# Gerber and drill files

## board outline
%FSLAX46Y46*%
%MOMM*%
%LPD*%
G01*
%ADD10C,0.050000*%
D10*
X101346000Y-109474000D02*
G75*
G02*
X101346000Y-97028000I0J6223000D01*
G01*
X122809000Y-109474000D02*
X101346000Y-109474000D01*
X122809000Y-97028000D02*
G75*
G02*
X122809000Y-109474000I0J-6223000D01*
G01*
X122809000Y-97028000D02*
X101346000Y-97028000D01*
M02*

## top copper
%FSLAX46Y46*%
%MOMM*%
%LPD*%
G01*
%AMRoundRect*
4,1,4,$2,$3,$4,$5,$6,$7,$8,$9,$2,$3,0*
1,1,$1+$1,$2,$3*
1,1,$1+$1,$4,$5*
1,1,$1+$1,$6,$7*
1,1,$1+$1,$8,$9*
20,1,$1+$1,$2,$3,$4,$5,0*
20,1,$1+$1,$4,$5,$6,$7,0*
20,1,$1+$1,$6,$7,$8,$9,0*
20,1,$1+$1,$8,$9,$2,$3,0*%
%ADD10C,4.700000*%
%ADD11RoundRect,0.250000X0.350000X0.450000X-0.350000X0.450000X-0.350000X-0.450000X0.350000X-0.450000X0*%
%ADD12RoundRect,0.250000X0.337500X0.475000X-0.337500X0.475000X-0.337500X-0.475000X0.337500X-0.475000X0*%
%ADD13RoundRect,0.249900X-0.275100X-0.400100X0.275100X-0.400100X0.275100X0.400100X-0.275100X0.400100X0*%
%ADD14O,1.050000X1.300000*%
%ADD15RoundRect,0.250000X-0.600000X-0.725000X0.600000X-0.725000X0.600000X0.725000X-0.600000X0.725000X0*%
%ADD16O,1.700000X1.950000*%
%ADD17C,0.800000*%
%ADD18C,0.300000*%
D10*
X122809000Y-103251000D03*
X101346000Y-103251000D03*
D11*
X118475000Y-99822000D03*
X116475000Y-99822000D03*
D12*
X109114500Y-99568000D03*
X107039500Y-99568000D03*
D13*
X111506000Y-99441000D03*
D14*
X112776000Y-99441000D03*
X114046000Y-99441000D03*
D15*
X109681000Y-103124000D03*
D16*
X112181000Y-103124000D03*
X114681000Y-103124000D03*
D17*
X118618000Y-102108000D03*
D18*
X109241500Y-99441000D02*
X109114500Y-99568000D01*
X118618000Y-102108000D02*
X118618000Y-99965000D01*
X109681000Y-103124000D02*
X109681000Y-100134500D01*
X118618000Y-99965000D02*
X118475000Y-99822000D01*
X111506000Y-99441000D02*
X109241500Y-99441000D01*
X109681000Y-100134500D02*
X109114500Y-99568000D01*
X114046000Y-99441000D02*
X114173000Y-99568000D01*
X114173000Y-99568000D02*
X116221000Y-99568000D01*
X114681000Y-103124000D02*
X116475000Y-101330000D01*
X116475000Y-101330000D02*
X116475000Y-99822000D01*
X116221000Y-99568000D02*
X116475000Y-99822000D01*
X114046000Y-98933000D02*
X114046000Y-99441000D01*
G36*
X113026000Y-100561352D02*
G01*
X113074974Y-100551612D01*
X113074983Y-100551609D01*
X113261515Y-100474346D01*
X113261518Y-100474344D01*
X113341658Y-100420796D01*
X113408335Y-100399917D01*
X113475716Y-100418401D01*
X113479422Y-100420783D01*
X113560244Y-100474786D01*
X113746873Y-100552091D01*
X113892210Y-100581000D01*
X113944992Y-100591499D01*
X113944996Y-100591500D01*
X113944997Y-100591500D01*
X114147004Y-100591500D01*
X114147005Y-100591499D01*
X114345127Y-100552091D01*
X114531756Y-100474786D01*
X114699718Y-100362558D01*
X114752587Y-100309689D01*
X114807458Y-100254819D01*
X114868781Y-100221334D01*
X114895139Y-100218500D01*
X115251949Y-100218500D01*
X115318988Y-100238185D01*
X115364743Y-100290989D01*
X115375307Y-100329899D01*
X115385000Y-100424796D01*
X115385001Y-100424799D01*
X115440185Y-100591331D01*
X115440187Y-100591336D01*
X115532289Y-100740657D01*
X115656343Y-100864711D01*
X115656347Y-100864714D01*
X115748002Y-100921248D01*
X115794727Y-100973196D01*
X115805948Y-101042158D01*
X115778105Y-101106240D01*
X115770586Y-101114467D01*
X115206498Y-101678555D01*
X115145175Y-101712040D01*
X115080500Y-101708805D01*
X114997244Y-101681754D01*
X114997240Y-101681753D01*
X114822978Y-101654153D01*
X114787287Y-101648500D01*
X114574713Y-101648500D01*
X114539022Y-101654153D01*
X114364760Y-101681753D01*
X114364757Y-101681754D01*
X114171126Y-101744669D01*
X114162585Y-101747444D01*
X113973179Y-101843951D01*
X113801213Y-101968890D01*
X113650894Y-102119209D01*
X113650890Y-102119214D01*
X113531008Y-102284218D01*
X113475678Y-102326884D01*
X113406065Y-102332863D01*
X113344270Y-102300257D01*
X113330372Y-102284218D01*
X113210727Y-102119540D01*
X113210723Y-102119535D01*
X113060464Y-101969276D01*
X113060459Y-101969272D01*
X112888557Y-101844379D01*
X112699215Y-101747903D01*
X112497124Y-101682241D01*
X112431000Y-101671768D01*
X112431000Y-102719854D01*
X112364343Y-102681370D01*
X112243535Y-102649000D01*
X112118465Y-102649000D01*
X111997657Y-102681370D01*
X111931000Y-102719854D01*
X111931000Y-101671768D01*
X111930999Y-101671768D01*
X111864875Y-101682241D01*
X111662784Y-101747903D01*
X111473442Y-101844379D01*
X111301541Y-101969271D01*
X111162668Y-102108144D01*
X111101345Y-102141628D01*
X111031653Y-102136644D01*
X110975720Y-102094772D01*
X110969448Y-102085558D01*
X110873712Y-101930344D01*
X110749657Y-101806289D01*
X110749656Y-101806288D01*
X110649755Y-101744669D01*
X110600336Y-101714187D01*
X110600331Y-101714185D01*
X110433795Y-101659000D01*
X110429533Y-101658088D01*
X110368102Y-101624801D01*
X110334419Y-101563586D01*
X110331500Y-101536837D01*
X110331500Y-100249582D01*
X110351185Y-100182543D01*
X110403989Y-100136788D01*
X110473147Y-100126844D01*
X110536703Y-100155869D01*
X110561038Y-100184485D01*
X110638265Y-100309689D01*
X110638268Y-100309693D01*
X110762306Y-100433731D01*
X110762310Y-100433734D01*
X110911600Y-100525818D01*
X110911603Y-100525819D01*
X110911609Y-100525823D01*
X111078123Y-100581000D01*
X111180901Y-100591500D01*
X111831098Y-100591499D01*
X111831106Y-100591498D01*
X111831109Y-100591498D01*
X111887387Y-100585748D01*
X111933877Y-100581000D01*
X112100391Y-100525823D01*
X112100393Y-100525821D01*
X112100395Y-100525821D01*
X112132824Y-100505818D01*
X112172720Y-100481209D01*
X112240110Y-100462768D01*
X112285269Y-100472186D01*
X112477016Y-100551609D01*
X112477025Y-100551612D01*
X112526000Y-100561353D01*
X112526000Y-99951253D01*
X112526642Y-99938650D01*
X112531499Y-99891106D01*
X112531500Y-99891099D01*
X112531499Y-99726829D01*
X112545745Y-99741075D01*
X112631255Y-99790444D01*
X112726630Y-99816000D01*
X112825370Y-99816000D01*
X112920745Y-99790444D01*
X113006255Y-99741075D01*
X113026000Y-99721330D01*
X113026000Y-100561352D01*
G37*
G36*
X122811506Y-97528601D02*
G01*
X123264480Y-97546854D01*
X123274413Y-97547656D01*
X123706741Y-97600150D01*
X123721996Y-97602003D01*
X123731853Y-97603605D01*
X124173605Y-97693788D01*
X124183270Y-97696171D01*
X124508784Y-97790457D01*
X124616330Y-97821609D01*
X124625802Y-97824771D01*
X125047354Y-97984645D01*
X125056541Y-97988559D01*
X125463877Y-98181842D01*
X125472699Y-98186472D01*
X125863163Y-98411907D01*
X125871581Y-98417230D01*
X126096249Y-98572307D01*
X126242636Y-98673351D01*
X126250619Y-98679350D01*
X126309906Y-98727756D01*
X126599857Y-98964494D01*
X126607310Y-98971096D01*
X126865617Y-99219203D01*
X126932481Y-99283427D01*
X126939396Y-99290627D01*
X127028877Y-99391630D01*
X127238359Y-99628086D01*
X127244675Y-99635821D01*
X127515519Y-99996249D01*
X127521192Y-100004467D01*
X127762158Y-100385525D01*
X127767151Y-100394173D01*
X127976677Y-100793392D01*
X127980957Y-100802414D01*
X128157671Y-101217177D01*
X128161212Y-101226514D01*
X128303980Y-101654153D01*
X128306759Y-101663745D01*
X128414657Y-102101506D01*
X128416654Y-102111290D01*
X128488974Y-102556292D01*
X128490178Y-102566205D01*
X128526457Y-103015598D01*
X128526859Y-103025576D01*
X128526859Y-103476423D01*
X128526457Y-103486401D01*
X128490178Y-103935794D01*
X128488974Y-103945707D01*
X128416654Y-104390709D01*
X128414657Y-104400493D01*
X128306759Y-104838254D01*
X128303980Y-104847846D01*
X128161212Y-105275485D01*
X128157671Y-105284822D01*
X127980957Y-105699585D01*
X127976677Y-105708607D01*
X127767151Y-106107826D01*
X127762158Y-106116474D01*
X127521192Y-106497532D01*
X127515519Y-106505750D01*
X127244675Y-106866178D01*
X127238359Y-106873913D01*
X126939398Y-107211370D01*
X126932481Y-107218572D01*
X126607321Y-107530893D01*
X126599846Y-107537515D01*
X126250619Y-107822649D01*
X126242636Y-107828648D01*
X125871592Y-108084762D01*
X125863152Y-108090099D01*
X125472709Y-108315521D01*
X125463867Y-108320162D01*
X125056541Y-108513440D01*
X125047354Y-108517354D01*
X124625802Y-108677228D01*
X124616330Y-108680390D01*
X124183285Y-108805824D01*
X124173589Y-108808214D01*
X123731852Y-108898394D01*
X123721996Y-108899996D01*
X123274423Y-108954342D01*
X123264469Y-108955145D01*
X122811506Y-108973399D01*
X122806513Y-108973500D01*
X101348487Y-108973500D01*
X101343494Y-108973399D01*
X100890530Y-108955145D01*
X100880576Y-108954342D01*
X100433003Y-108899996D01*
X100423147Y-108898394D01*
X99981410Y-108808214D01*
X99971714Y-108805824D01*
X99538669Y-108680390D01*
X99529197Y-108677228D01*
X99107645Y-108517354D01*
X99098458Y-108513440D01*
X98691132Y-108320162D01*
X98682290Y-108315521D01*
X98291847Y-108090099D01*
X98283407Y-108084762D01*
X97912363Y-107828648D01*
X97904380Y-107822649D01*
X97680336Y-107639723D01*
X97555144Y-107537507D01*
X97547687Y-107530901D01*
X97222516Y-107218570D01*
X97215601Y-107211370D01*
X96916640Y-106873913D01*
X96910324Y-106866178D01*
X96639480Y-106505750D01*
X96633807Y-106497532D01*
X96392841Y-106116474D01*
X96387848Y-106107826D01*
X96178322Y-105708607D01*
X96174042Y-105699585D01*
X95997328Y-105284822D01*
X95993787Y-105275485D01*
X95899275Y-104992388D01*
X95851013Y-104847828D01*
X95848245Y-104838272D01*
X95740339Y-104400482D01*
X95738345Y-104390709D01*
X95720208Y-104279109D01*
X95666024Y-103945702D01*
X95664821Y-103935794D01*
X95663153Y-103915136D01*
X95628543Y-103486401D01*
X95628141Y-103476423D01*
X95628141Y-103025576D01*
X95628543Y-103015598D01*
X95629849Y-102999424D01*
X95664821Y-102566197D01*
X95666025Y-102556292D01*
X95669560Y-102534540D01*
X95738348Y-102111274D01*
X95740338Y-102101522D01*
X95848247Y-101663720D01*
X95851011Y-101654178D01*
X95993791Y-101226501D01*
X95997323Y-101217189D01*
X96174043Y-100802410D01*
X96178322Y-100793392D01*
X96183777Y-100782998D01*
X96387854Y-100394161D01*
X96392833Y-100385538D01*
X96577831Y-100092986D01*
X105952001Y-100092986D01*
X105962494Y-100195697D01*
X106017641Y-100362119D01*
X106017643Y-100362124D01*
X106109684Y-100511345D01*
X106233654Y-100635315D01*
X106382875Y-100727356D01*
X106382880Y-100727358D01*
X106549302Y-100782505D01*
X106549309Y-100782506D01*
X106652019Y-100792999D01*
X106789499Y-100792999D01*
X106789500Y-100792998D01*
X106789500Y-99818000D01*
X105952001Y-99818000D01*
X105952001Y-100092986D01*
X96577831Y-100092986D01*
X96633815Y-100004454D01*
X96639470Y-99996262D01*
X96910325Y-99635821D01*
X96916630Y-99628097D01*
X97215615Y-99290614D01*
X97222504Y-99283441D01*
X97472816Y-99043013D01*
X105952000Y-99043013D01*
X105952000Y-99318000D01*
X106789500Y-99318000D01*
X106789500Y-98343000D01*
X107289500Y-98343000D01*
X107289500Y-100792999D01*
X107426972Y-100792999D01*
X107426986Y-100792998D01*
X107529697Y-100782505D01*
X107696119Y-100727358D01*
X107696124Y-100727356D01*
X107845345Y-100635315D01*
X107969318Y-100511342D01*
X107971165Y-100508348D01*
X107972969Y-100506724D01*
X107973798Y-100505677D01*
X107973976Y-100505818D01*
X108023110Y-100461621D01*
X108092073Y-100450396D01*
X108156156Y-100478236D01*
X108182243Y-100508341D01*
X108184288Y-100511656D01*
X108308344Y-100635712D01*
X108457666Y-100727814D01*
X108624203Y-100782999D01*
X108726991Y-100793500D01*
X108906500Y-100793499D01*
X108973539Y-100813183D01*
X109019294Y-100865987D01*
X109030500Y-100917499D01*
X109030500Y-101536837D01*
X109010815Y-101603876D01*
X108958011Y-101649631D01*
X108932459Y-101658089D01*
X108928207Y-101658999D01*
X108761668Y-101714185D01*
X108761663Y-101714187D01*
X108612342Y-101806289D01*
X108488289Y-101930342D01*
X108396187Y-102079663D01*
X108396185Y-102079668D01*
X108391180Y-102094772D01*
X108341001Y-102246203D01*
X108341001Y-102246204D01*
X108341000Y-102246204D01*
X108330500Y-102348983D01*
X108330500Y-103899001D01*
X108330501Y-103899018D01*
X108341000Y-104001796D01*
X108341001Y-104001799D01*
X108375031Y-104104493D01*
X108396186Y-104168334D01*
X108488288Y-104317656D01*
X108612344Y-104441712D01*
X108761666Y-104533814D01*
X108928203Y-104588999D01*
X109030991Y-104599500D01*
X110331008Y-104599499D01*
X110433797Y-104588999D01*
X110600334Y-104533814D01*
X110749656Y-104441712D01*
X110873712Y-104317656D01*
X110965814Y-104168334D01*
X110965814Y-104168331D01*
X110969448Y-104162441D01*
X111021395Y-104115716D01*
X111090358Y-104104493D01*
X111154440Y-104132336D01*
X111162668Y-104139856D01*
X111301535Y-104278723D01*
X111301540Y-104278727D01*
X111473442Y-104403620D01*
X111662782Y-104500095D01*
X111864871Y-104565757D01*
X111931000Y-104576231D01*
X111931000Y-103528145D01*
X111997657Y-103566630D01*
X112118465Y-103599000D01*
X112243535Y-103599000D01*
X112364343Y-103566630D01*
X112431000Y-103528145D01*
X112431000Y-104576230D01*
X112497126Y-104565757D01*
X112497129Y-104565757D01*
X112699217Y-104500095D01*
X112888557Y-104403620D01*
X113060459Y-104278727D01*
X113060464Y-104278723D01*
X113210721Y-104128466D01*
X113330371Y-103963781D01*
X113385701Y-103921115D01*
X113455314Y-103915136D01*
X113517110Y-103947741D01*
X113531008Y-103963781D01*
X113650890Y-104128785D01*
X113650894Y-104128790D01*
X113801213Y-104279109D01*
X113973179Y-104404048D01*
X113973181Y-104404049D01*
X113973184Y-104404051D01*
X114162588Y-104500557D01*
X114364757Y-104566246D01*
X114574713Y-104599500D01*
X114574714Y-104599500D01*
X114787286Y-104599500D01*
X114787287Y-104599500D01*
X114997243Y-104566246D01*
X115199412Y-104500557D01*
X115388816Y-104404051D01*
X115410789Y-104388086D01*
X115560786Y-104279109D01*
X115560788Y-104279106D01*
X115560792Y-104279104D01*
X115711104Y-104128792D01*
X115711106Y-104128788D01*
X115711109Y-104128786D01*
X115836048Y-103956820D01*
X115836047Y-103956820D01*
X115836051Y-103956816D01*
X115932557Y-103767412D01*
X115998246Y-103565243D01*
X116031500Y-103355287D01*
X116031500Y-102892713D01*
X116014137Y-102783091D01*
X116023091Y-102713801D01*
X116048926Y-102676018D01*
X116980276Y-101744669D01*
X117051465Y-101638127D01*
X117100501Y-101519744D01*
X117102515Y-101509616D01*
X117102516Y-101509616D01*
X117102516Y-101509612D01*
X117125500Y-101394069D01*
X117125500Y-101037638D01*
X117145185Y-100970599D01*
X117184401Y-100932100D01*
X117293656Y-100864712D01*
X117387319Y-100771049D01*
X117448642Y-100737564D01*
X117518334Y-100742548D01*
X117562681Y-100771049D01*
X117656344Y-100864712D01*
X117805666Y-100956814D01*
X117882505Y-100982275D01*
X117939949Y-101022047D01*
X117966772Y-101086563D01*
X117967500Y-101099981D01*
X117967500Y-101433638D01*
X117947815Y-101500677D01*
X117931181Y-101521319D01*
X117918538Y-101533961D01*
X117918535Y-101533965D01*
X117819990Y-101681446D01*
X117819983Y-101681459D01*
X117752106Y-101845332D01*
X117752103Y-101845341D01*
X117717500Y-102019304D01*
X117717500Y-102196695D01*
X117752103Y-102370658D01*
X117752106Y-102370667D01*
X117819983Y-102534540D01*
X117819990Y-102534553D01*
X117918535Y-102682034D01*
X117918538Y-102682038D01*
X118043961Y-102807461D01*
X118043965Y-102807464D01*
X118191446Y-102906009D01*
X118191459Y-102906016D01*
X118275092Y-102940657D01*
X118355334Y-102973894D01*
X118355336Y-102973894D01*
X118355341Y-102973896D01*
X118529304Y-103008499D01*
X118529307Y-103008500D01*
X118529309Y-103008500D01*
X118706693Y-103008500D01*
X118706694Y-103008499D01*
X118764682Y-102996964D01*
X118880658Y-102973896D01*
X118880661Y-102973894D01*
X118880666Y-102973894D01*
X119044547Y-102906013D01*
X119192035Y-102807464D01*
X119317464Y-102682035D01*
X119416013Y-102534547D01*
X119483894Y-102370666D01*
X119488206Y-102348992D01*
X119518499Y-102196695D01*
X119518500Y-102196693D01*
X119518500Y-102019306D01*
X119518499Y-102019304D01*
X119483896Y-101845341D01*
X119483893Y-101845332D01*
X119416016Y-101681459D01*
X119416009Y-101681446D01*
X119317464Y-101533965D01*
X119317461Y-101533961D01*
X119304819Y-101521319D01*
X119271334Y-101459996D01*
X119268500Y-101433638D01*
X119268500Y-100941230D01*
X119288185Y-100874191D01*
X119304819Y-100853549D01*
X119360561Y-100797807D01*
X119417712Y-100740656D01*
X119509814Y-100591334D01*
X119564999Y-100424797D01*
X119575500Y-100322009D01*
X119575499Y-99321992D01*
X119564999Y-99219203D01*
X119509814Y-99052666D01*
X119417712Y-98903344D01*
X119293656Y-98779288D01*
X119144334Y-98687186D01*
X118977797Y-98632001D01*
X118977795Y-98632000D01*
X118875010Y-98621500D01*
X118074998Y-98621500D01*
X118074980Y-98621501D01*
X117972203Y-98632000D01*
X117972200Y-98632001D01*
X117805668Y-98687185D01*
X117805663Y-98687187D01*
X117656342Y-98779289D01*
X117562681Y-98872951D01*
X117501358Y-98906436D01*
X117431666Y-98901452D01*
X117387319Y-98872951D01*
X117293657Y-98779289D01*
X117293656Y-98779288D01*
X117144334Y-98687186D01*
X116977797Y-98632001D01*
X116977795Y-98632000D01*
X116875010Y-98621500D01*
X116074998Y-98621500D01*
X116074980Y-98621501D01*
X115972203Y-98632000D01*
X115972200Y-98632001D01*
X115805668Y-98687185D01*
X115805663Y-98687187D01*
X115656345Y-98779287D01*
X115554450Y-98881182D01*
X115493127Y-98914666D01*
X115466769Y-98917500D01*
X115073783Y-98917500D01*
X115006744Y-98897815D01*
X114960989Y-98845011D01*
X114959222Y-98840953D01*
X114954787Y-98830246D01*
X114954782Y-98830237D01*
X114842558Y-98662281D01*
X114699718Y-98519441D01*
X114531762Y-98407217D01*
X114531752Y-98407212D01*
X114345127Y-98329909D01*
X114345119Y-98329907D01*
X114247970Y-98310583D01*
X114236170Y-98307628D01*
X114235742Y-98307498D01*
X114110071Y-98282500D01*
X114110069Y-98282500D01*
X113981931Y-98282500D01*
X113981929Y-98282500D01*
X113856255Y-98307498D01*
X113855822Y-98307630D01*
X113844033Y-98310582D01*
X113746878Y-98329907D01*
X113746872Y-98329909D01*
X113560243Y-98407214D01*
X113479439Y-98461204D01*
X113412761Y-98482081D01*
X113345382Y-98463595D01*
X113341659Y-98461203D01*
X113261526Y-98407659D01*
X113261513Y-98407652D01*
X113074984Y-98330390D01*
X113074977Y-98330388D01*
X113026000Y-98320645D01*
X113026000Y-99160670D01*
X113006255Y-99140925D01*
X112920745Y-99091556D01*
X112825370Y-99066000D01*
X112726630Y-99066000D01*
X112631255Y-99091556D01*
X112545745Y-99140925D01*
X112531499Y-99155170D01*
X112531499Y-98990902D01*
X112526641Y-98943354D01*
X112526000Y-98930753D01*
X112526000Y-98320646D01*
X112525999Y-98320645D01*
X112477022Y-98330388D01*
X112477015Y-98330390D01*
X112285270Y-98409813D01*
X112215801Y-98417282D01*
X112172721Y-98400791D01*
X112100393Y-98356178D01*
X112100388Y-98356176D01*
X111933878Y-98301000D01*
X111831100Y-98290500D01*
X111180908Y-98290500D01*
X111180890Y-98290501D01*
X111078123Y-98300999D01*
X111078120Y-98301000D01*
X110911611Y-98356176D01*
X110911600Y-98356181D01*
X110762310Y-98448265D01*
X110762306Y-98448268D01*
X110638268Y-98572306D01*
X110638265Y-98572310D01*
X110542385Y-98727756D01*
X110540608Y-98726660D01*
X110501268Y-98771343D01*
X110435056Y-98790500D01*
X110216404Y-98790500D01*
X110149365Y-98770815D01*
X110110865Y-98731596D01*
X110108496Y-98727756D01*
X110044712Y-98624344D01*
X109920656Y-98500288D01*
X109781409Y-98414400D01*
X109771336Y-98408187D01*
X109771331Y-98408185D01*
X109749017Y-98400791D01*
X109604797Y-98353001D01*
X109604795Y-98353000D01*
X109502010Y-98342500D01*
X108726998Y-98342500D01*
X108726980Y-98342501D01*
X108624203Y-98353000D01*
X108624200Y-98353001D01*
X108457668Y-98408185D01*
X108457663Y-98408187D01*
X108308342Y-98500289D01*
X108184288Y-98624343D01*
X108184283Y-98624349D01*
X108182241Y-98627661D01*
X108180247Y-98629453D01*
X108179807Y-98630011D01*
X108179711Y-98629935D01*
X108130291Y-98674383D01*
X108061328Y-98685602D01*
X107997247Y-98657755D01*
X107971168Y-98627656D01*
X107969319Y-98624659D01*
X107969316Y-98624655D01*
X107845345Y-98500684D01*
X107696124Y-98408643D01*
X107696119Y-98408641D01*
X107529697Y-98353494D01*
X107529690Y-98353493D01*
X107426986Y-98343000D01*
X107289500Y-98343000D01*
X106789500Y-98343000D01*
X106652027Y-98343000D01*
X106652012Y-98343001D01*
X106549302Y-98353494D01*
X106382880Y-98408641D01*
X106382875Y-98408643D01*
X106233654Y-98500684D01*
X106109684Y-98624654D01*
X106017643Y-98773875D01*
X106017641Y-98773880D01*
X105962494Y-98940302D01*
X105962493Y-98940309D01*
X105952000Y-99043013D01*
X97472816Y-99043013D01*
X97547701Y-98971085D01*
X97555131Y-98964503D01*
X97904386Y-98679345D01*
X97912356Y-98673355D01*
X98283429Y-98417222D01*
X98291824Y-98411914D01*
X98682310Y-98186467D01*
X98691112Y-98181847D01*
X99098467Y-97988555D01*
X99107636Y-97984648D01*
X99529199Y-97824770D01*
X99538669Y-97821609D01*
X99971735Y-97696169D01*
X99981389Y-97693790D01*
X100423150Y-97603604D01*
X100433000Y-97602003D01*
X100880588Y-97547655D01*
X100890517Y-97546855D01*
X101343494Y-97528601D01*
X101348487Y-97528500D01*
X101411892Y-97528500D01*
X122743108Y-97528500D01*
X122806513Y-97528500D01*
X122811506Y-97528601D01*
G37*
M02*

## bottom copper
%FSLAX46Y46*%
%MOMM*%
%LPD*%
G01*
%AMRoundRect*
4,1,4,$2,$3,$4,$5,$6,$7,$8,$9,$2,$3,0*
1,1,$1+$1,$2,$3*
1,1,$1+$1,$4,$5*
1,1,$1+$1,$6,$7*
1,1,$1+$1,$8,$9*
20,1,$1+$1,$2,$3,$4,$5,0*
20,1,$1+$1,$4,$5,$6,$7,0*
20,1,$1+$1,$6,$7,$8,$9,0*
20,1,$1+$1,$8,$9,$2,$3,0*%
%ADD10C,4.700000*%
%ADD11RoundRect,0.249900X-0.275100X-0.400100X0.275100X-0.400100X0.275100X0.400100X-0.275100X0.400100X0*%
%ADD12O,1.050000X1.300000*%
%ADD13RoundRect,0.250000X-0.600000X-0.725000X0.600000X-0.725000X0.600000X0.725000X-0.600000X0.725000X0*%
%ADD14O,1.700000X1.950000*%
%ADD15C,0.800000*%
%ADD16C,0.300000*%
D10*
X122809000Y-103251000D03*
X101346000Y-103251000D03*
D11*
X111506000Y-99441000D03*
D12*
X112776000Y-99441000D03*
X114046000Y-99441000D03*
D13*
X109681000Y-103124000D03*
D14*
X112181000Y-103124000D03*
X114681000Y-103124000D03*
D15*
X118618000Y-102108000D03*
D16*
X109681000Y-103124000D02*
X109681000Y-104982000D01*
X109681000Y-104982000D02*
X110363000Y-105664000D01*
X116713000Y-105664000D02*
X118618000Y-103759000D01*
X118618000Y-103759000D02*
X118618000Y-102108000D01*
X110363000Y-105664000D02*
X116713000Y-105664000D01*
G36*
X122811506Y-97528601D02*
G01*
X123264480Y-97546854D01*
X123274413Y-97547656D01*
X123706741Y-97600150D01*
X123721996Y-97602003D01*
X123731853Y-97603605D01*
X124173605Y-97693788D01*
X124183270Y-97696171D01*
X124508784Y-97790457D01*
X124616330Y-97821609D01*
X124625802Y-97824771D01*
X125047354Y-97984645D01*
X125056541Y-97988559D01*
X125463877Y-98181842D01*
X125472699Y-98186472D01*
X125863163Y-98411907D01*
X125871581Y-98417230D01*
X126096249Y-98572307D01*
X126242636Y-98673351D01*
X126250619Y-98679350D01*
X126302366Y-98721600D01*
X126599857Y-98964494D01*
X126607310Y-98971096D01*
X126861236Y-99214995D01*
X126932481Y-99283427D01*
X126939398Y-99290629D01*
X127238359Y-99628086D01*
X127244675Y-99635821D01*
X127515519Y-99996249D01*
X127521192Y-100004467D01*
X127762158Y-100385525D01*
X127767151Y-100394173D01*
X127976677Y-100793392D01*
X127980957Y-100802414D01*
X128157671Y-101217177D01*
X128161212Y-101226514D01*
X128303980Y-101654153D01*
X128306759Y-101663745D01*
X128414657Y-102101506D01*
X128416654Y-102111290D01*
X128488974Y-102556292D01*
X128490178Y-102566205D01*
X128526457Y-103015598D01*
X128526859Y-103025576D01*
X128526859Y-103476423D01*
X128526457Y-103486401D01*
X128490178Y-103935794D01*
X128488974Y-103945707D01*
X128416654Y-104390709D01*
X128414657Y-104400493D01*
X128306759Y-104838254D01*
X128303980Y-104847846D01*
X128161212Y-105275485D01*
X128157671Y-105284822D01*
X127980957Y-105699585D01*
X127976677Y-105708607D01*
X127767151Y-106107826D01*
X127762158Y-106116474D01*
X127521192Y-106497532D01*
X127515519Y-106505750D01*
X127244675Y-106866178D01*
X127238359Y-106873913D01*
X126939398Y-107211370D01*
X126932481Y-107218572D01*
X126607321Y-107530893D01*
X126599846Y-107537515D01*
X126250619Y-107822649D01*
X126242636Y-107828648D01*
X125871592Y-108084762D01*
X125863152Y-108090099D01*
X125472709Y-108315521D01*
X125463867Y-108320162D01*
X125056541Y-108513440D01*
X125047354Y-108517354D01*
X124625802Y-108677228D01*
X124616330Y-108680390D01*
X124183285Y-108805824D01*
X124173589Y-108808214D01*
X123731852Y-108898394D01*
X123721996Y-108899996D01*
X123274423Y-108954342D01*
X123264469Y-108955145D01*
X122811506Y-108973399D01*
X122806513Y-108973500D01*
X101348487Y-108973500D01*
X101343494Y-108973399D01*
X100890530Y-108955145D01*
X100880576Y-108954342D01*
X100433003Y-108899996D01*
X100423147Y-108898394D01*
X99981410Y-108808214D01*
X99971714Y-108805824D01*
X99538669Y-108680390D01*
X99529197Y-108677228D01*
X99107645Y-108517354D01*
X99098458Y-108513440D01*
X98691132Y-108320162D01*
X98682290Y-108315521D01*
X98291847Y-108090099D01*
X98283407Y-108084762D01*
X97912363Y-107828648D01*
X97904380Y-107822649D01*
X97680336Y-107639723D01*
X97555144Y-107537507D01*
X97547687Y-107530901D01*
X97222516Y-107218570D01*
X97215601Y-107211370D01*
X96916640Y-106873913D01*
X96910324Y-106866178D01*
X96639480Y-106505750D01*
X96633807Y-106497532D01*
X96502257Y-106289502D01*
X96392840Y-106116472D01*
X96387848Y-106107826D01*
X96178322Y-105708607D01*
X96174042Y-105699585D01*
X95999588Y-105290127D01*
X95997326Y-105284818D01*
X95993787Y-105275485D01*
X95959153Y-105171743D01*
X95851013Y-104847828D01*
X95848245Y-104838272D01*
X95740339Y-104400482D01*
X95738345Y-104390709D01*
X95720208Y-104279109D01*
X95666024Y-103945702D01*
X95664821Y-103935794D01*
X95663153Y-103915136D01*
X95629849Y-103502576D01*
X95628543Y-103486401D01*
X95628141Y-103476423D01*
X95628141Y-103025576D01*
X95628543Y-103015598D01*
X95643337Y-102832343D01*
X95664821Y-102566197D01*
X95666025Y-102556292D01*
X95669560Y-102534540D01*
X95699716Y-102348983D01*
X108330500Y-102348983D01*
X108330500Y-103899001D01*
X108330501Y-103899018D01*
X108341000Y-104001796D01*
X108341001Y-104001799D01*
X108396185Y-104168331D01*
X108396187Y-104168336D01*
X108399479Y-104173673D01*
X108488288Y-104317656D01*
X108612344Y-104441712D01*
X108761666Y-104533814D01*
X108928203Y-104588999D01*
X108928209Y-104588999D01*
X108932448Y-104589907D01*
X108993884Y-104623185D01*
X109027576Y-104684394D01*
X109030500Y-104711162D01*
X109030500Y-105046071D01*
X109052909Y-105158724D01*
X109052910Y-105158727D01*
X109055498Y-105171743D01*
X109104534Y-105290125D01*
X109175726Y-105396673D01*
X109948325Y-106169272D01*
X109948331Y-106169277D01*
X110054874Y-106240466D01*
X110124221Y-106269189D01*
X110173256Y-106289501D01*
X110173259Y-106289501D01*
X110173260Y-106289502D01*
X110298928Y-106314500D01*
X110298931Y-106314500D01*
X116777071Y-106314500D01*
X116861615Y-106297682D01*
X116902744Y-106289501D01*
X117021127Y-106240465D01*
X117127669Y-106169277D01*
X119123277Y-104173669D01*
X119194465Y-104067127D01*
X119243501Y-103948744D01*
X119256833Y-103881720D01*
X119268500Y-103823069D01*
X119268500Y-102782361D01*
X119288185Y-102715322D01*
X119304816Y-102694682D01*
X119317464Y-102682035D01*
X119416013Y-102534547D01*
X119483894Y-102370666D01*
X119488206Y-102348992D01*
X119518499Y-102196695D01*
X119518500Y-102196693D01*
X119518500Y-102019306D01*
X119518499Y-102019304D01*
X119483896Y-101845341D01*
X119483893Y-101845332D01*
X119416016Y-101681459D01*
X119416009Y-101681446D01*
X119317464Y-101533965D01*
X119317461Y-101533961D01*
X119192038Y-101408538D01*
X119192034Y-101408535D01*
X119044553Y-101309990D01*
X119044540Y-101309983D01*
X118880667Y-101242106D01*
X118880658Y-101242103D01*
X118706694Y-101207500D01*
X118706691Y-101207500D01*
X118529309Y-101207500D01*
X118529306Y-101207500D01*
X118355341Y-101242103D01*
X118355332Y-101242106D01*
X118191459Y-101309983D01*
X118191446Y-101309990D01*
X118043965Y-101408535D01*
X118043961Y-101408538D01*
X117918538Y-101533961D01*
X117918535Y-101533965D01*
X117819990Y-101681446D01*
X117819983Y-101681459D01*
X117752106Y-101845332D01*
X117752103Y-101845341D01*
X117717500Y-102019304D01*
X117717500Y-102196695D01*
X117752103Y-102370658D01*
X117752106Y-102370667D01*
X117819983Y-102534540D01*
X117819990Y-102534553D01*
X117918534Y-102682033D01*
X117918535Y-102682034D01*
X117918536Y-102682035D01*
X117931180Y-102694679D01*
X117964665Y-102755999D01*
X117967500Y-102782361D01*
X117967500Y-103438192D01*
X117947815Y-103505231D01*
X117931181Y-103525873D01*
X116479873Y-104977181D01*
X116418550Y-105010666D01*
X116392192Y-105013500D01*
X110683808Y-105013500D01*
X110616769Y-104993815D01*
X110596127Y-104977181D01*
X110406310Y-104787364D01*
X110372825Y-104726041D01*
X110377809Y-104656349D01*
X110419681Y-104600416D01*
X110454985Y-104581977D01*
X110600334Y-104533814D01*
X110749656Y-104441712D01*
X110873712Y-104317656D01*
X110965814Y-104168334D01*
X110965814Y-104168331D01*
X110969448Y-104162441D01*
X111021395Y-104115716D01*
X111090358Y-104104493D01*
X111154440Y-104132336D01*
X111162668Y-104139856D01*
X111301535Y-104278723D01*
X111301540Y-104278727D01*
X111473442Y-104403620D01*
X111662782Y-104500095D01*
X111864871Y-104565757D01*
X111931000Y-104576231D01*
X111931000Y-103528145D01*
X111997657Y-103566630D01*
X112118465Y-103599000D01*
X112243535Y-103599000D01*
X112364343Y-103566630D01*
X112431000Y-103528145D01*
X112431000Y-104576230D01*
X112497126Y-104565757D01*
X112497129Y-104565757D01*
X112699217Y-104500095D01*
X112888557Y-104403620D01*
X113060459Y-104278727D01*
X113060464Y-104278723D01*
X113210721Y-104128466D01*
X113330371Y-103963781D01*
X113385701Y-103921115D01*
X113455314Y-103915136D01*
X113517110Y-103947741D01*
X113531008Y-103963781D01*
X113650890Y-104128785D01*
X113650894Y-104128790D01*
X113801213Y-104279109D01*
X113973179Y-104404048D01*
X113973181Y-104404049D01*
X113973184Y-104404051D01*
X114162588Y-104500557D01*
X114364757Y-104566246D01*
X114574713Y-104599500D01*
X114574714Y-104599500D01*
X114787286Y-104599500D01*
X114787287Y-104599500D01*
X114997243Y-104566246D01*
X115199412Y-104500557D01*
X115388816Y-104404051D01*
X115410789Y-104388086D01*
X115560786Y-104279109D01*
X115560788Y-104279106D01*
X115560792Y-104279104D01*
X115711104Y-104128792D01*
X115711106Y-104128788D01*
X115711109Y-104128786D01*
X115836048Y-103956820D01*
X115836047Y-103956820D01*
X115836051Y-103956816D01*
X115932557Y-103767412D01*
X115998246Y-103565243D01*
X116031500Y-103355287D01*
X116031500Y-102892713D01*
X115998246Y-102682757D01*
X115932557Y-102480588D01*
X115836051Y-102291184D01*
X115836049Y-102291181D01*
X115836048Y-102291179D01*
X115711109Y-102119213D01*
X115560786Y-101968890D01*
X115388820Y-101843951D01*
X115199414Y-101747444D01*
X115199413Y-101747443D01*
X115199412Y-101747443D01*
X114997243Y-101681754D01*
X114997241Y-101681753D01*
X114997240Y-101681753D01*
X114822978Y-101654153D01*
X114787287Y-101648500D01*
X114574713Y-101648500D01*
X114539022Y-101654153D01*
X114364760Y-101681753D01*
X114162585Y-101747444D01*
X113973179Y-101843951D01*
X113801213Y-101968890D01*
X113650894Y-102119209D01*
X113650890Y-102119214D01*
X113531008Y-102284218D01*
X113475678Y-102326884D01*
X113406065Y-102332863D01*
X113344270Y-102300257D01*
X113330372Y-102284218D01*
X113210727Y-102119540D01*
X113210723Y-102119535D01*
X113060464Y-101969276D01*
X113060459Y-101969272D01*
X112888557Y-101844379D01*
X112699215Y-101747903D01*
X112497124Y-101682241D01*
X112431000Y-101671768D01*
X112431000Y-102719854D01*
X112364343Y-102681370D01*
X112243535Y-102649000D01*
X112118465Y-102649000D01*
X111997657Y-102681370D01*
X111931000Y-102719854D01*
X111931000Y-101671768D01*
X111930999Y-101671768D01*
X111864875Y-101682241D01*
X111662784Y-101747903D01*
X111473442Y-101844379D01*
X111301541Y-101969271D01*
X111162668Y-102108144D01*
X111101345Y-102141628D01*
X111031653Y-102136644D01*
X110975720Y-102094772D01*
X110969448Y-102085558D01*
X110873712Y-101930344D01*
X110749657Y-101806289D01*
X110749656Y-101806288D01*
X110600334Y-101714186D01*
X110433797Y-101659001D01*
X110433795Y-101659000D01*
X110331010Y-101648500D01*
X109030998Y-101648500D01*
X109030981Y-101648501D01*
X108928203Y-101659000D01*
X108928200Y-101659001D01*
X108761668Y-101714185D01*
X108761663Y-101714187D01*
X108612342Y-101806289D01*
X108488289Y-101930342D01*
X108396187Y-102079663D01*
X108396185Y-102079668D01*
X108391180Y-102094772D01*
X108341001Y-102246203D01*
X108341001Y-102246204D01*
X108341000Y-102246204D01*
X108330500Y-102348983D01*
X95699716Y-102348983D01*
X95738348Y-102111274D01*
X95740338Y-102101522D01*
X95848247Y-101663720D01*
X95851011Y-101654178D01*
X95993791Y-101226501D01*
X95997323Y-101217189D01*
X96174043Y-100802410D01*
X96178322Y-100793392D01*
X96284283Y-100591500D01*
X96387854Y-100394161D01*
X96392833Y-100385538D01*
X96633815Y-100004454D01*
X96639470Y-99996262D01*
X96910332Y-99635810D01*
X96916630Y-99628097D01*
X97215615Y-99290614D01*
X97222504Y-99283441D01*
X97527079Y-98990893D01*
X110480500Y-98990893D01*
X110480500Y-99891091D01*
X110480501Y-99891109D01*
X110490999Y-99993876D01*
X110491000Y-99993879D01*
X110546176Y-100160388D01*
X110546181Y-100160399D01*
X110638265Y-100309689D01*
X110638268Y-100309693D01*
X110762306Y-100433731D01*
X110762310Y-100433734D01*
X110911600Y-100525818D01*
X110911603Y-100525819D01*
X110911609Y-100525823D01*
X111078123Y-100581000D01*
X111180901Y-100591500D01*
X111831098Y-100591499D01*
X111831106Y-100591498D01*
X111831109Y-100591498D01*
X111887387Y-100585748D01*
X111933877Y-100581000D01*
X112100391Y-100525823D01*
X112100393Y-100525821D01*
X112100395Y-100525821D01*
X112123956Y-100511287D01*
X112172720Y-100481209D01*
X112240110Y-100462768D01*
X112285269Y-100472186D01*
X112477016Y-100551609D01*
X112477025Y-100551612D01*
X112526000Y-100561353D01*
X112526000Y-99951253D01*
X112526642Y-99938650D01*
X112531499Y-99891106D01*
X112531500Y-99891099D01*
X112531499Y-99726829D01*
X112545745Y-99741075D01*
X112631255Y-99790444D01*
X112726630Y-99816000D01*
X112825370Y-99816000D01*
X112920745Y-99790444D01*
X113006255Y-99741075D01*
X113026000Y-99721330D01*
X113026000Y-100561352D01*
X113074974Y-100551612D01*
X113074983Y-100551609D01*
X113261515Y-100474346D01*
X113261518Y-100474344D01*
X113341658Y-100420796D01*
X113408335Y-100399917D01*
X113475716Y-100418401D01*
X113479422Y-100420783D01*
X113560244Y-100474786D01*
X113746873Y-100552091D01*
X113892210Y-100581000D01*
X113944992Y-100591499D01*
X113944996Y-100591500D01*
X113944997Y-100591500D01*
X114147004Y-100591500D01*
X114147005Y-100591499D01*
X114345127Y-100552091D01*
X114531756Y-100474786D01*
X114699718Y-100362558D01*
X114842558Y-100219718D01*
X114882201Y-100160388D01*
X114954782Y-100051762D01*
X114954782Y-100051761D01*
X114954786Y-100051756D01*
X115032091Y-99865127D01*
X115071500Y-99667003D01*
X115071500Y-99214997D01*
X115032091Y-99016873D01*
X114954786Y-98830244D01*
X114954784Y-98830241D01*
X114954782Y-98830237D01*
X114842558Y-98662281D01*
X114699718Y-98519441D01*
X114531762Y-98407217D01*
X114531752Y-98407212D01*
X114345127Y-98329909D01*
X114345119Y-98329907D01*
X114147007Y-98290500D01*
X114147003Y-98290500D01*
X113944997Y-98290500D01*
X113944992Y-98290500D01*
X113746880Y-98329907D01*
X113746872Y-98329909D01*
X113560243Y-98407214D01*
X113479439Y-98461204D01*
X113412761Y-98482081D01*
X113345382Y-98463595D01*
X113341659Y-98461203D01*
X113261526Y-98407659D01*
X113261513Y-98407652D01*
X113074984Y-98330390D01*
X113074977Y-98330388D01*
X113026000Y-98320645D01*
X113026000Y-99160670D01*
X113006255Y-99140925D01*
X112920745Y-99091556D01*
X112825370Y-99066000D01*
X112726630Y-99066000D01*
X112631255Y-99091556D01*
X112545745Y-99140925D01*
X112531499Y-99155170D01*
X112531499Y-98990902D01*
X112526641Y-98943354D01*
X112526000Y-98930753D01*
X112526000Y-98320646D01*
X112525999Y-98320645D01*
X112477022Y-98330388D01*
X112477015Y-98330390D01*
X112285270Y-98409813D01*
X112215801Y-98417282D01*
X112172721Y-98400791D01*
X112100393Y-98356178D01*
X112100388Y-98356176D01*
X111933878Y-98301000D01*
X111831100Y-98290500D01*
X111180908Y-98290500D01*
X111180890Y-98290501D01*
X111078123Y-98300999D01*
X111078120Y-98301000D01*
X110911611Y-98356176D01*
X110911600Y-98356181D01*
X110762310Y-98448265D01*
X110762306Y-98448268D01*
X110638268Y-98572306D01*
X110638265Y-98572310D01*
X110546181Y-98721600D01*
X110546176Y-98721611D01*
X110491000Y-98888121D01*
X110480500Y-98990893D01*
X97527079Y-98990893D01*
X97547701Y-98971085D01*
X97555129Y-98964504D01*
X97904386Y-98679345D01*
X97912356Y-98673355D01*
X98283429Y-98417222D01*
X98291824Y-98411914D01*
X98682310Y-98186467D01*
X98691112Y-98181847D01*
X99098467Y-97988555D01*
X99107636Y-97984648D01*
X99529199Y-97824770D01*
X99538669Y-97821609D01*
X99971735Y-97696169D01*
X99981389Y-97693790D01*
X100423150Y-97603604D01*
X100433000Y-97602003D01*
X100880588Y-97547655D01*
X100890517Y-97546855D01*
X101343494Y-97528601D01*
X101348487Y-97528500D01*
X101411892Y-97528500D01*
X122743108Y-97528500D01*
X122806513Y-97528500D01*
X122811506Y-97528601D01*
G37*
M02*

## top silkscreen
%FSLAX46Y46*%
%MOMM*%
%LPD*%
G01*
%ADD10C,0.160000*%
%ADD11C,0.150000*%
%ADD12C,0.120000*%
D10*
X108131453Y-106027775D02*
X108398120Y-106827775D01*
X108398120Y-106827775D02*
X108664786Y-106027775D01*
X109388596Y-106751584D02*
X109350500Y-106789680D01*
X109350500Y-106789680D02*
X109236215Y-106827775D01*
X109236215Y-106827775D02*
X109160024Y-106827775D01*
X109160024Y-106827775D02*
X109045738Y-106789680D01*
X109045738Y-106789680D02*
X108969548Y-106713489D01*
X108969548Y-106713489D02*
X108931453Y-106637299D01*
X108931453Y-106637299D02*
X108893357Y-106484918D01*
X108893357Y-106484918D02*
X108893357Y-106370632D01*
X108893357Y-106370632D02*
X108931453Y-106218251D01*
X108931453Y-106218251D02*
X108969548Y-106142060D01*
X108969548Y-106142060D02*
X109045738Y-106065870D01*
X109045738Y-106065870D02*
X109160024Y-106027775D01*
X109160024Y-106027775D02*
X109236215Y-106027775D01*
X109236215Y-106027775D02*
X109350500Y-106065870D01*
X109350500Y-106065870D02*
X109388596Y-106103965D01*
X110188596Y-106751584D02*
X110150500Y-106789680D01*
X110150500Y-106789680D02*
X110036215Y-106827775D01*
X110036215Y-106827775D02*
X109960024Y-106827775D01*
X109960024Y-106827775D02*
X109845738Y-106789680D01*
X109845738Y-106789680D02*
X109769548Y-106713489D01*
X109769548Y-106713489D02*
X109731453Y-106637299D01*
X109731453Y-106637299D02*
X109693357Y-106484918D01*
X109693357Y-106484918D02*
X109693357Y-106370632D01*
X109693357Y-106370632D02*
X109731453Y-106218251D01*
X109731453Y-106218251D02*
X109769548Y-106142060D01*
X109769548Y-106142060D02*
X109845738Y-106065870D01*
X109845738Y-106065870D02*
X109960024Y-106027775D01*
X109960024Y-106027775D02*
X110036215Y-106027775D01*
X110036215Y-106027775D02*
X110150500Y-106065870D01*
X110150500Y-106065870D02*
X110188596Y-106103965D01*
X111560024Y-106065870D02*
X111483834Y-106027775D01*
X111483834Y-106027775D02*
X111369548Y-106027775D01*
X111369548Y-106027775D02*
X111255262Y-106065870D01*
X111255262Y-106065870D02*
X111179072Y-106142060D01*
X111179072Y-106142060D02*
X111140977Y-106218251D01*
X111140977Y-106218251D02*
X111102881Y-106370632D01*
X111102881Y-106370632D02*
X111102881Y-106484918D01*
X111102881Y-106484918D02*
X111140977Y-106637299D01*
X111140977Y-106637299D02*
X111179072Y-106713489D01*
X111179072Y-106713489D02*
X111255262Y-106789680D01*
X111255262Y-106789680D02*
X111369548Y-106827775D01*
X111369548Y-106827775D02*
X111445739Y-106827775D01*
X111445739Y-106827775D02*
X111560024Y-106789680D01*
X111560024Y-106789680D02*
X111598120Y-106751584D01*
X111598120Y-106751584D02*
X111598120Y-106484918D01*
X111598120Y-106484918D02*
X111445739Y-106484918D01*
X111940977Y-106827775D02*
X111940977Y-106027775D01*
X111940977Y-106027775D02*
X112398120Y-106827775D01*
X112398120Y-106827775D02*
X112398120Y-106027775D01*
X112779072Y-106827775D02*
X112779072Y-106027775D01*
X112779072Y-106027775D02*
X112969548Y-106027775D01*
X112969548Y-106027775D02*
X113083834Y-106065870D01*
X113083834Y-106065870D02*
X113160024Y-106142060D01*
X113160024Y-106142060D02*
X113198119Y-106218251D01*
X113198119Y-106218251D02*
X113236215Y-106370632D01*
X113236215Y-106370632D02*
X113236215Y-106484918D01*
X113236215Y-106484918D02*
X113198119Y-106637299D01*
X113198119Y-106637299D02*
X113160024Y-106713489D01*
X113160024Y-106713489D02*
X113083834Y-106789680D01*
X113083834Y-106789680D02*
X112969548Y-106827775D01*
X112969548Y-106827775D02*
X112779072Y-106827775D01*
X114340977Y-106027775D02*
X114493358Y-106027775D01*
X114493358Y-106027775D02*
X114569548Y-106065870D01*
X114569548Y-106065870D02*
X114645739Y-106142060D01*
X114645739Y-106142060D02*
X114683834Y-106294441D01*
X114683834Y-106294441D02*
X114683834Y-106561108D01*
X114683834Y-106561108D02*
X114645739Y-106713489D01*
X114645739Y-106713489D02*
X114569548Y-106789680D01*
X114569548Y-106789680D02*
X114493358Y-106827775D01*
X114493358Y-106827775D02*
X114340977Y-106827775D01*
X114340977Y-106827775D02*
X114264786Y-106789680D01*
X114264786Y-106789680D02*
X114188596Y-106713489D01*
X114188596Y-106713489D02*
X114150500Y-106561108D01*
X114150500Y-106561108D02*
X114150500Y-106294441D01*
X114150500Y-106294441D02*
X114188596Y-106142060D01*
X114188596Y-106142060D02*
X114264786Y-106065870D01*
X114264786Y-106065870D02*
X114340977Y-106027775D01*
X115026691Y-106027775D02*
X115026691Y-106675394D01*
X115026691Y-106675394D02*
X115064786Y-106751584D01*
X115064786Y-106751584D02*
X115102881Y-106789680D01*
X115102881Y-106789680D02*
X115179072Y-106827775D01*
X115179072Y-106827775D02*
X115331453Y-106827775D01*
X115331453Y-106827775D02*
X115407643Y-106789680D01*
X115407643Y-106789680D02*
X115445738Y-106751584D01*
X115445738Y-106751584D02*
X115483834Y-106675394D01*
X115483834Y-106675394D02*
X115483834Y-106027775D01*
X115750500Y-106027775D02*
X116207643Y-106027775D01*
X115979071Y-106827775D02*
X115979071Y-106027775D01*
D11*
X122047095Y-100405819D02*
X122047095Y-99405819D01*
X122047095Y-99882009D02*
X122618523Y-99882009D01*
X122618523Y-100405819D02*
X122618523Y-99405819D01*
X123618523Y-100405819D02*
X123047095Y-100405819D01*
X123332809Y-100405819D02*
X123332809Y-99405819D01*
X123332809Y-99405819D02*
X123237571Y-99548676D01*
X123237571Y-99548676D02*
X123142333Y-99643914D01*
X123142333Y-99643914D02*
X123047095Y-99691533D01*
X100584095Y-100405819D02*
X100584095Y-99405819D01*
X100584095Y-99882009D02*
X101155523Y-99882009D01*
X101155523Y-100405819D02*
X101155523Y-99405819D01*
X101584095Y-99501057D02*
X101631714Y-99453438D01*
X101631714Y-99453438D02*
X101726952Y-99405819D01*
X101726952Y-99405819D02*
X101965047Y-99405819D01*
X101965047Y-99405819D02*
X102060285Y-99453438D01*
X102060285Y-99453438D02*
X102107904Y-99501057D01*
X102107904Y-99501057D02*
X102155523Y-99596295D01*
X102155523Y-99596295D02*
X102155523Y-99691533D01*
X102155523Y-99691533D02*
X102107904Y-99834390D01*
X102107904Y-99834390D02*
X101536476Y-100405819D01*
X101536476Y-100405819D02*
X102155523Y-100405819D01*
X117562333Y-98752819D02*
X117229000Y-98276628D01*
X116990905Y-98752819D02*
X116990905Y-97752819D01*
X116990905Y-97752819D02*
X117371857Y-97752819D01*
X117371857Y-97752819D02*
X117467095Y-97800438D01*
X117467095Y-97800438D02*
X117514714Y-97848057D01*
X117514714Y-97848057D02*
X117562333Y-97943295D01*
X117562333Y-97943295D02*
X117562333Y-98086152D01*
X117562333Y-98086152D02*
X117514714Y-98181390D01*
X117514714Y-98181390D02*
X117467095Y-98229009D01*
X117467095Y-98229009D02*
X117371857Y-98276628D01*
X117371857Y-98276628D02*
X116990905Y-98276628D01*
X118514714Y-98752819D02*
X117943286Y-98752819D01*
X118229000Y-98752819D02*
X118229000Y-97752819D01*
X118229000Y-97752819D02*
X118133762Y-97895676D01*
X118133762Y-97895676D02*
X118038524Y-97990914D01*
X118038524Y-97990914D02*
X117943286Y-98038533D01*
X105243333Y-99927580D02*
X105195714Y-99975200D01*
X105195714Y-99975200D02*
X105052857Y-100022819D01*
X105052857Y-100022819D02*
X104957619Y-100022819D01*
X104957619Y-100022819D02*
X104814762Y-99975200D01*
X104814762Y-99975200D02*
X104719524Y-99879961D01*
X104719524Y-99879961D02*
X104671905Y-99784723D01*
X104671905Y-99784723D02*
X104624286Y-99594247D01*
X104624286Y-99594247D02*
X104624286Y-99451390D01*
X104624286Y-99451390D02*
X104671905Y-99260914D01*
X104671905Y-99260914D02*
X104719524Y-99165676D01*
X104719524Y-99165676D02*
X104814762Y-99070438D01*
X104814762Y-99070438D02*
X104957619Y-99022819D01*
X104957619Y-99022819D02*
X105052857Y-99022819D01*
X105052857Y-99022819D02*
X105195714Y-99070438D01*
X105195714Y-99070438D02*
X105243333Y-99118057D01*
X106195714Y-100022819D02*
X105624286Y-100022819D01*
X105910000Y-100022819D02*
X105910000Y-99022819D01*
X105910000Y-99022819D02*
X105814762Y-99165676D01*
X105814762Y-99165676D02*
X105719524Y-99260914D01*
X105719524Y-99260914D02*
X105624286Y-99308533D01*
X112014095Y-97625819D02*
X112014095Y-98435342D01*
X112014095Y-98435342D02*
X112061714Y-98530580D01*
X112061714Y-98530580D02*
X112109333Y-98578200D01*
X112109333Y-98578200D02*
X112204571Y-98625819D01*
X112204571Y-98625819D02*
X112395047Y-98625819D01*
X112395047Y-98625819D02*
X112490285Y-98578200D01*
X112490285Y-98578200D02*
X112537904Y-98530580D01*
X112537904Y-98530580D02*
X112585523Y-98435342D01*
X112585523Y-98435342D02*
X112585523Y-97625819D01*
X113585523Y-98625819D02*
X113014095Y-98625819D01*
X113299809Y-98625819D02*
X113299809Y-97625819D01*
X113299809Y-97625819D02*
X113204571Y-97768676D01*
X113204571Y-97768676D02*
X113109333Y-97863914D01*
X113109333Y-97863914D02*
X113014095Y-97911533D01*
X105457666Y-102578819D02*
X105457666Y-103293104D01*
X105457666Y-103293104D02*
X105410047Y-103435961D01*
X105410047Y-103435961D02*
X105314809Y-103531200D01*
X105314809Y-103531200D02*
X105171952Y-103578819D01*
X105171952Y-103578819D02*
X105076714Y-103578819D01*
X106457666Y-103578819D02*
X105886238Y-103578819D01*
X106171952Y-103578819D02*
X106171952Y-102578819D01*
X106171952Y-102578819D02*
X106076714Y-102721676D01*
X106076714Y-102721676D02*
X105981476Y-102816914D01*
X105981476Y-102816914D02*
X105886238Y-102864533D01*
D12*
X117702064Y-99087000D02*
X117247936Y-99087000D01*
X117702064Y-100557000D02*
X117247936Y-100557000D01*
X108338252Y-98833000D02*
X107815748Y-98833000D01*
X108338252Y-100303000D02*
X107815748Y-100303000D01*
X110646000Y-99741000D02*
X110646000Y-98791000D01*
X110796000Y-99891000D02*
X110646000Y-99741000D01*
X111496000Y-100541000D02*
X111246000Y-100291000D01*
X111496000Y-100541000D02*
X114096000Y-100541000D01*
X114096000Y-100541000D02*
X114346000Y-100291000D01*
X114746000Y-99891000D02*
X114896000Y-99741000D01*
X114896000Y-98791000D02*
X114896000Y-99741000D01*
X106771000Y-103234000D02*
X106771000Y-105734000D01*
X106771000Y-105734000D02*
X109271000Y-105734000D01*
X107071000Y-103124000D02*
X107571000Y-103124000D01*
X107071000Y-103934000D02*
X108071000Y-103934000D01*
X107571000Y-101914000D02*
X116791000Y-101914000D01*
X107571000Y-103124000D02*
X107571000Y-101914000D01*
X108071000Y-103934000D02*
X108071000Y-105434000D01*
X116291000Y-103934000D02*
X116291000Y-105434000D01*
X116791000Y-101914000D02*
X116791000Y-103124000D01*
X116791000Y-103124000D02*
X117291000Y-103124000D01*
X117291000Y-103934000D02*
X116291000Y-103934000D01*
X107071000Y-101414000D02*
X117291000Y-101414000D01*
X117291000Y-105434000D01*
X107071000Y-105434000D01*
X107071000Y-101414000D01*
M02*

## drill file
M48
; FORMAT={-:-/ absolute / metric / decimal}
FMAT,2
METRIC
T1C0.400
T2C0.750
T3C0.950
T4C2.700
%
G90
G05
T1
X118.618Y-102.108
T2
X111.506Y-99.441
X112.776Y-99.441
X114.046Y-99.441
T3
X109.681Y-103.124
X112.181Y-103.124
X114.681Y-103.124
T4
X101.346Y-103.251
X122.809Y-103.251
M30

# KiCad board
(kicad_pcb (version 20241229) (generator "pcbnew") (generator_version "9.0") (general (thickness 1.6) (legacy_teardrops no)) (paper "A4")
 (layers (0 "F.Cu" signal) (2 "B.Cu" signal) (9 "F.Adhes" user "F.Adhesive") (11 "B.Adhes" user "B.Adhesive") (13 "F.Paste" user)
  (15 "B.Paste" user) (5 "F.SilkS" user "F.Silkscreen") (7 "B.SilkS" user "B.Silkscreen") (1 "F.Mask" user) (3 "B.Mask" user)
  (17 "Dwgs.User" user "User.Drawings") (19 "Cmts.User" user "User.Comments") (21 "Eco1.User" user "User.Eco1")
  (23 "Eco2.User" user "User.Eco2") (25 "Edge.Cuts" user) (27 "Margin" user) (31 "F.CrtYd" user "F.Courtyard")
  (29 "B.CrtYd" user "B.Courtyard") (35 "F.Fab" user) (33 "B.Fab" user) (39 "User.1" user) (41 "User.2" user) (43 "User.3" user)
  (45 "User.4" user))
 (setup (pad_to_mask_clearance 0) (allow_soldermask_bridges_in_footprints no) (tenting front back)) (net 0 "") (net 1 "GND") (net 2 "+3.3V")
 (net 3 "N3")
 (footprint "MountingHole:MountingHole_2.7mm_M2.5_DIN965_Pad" (layer "F.Cu") (at 122.809 103.251)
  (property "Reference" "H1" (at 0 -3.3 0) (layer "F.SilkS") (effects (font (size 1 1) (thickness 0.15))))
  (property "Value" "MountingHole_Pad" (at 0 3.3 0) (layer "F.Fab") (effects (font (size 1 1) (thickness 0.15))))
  (pad "1" thru_hole circle (at 0 0) (size 4.7 4.7) (drill 2.7) (layers "*.Cu" "*.Mask") (remove_unused_layers no) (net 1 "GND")
   (zone_connect 2)))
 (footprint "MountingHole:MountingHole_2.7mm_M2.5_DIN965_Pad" (layer "F.Cu") (at 101.346 103.251)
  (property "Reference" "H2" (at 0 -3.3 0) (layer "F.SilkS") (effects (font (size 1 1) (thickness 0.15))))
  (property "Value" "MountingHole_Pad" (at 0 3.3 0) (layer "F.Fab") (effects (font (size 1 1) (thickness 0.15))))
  (pad "1" thru_hole circle (at 0 0) (size 4.7 4.7) (drill 2.7) (layers "*.Cu" "*.Mask") (remove_unused_layers no) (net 1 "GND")
   (zone_connect 2)))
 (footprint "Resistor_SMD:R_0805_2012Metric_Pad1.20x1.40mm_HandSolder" (layer "F.Cu") (at 117.475 99.822 180)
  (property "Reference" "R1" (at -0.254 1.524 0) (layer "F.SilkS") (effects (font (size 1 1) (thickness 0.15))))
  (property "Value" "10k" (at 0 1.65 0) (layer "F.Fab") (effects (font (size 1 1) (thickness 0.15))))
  (fp_line (start -0.227064 0.735) (end 0.227064 0.735) (stroke (width 0.12) (type solid)) (layer "F.SilkS"))
  (fp_line (start -0.227064 -0.735) (end 0.227064 -0.735) (stroke (width 0.12) (type solid)) (layer "F.SilkS"))
  (pad "1" smd roundrect (at -1 0 180) (size 1.2 1.4) (layers "F.Cu" "F.Mask" "F.Paste") (roundrect_rratio 0.208333) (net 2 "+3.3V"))
  (pad "2" smd roundrect (at 1 0 180) (size 1.2 1.4) (layers "F.Cu" "F.Mask" "F.Paste") (roundrect_rratio 0.208333) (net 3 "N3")))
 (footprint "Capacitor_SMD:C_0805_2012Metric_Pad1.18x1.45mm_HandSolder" (layer "F.Cu") (at 108.077 99.568 180)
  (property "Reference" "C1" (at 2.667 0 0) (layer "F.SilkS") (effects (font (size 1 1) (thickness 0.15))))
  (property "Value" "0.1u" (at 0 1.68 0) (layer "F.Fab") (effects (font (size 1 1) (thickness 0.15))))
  (fp_line (start -0.261252 0.735) (end 0.261252 0.735) (stroke (width 0.12) (type solid)) (layer "F.SilkS"))
  (fp_line (start -0.261252 -0.735) (end 0.261252 -0.735) (stroke (width 0.12) (type solid)) (layer "F.SilkS"))
  (pad "1" smd roundrect (at -1.0375 0 180) (size 1.175 1.45) (layers "F.Cu" "F.Mask" "F.Paste") (roundrect_rratio 0.212766) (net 2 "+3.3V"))
  (pad "2" smd roundrect (at 1.0375 0 180) (size 1.175 1.45) (layers "F.Cu" "F.Mask" "F.Paste") (roundrect_rratio 0.212766) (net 1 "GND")))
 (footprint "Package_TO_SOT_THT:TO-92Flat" (layer "F.Cu") (at 111.506 99.441)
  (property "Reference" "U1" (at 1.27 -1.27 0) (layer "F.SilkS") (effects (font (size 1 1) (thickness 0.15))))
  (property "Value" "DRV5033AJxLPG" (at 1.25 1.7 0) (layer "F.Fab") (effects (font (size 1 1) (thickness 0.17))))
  (fp_line (start -0.86 0.3) (end -0.86 -0.65) (stroke (width 0.12) (type solid)) (layer "F.SilkS"))
  (fp_line (start -0.71 0.45) (end -0.86 0.3) (stroke (width 0.12) (type solid)) (layer "F.SilkS"))
  (fp_line (start -0.01 1.1) (end -0.26 0.85) (stroke (width 0.12) (type solid)) (layer "F.SilkS"))
  (fp_line (start -0.01 1.1) (end 2.59 1.1) (stroke (width 0.12) (type solid)) (layer "F.SilkS"))
  (fp_line (start 2.59 1.1) (end 2.84 0.85) (stroke (width 0.12) (type solid)) (layer "F.SilkS"))
  (fp_line (start 3.24 0.45) (end 3.39 0.3) (stroke (width 0.12) (type solid)) (layer "F.SilkS"))
  (fp_line (start 3.39 -0.65) (end 3.39 0.3) (stroke (width 0.12) (type solid)) (layer "F.SilkS"))
  (pad "1" thru_hole roundrect (at 0 0) (size 1.05 1.3) (drill 0.75) (layers "*.Cu" "*.Mask") (remove_unused_layers no)
   (roundrect_rratio 0.238) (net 2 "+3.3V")
   (teardrops (best_length_ratio 0.5) (max_length 1) (best_width_ratio 1) (max_width 1) (curved_edges no) (filter_ratio 0.9) (enabled no)
    (allow_two_segments yes) (prefer_zone_connections yes)))
  (pad "2" thru_hole oval (at 1.27 0) (size 1.05 1.3) (drill 0.75) (layers "*.Cu" "*.Mask") (remove_unused_layers no) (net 1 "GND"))
  (pad "3" thru_hole oval (at 2.54 0) (size 1.05 1.3) (drill 0.75) (layers "*.Cu" "*.Mask") (remove_unused_layers no) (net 3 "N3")))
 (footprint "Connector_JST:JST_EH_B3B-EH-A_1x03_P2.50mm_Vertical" (layer "F.Cu") (at 109.681 103.124)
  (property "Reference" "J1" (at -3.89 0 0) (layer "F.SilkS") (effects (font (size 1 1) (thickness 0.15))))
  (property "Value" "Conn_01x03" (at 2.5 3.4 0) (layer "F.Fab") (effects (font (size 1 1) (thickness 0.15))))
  (fp_line (start -2.91 0.11) (end -2.91 2.61) (stroke (width 0.12) (type solid)) (layer "F.SilkS"))
  (fp_line (start -2.91 2.61) (end -0.41 2.61) (stroke (width 0.12) (type solid)) (layer "F.SilkS"))
  (fp_line (start -2.61 0) (end -2.11 0) (stroke (width 0.12) (type solid)) (layer "F.SilkS"))
  (fp_line (start -2.61 0.81) (end -1.61 0.81) (stroke (width 0.12) (type solid)) (layer "F.SilkS"))
  (fp_line (start -2.11 -1.21) (end 7.11 -1.21) (stroke (width 0.12) (type solid)) (layer "F.SilkS"))
  (fp_line (start -2.11 0) (end -2.11 -1.21) (stroke (width 0.12) (type solid)) (layer "F.SilkS"))
  (fp_line (start -1.61 0.81) (end -1.61 2.31) (stroke (width 0.12) (type solid)) (layer "F.SilkS"))
  (fp_line (start 6.61 0.81) (end 6.61 2.31) (stroke (width 0.12) (type solid)) (layer "F.SilkS"))
  (fp_line (start 7.11 -1.21) (end 7.11 0) (stroke (width 0.12) (type solid)) (layer "F.SilkS"))
  (fp_line (start 7.11 0) (end 7.61 0) (stroke (width 0.12) (type solid)) (layer "F.SilkS"))
  (fp_line (start 7.61 0.81) (end 6.61 0.81) (stroke (width 0.12) (type solid)) (layer "F.SilkS"))
  (fp_rect (start -2.61 -1.71) (end 7.61 2.31) (stroke (width 0.12) (type solid)) (fill no) (layer "F.SilkS"))
  (pad "1" thru_hole roundrect (at 0 0) (size 1.7 1.95) (drill 0.95) (layers "*.Cu" "*.Mask") (remove_unused_layers no)
   (roundrect_rratio 0.147059) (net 2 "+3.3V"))
  (pad "2" thru_hole oval (at 2.5 0) (size 1.7 1.95) (drill 0.95) (layers "*.Cu" "*.Mask") (remove_unused_layers no) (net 1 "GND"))
  (pad "3" thru_hole oval (at 5 0) (size 1.7 1.95) (drill 0.95) (layers "*.Cu" "*.Mask") (remove_unused_layers no) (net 3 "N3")))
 (gr_arc (start 101.346 109.474) (mid 95.123 103.251) (end 101.346 97.028) (stroke (width 0.05) (type default)) (layer "Edge.Cuts"))
 (gr_line (start 122.809 109.474) (end 101.346 109.474) (stroke (width 0.05) (type default)) (layer "Edge.Cuts"))
 (gr_arc (start 122.809 97.028) (mid 129.032 103.251) (end 122.809 109.474) (stroke (width 0.05) (type default)) (layer "Edge.Cuts"))
 (gr_line (start 122.809 97.028) (end 101.346 97.028) (stroke (width 0.05) (type default)) (layer "Edge.Cuts"))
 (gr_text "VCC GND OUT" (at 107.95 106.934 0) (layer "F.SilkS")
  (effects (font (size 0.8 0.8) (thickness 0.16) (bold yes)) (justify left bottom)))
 (segment (start 109.2415 99.441) (end 109.1145 99.568) (width 0.3) (layer "F.Cu") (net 2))
 (segment (start 118.618 102.108) (end 118.618 99.965) (width 0.3) (layer "F.Cu") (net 2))
 (segment (start 109.681 103.124) (end 109.681 100.1345) (width 0.3) (layer "F.Cu") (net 2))
 (segment (start 118.618 99.965) (end 118.475 99.822) (width 0.3) (layer "F.Cu") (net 2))
 (segment (start 111.506 99.441) (end 109.2415 99.441) (width 0.3) (layer "F.Cu") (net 2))
 (segment (start 109.681 100.1345) (end 109.1145 99.568) (width 0.3) (layer "F.Cu") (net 2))
 (via (at 118.618 102.108) (size 0.8) (drill 0.4) (layers "F.Cu" "B.Cu") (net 2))
 (segment (start 109.681 103.124) (end 109.681 104.982) (width 0.3) (layer "B.Cu") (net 2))
 (segment (start 109.681 104.982) (end 110.363 105.664) (width 0.3) (layer "B.Cu") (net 2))
 (segment (start 116.713 105.664) (end 118.618 103.759) (width 0.3) (layer "B.Cu") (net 2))
 (segment (start 118.618 103.759) (end 118.618 102.108) (width 0.3) (layer "B.Cu") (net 2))
 (segment (start 110.363 105.664) (end 116.713 105.664) (width 0.3) (layer "B.Cu") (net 2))
 (segment (start 114.046 99.441) (end 114.173 99.568) (width 0.3) (layer "F.Cu") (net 3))
 (segment (start 114.173 99.568) (end 116.221 99.568) (width 0.3) (layer "F.Cu") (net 3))
 (segment (start 114.681 103.124) (end 116.475 101.33) (width 0.3) (layer "F.Cu") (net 3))
 (segment (start 116.475 101.33) (end 116.475 99.822) (width 0.3) (layer "F.Cu") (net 3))
 (segment (start 116.221 99.568) (end 116.475 99.822) (width 0.3) (layer "F.Cu") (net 3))
 (segment (start 114.046 98.933) (end 114.046 99.441) (width 0.3) (layer "F.Cu") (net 3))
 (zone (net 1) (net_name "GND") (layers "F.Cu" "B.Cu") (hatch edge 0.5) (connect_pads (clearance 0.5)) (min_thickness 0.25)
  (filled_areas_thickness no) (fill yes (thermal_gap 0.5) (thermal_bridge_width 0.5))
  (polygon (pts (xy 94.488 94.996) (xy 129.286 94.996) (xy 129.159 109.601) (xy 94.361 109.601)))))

